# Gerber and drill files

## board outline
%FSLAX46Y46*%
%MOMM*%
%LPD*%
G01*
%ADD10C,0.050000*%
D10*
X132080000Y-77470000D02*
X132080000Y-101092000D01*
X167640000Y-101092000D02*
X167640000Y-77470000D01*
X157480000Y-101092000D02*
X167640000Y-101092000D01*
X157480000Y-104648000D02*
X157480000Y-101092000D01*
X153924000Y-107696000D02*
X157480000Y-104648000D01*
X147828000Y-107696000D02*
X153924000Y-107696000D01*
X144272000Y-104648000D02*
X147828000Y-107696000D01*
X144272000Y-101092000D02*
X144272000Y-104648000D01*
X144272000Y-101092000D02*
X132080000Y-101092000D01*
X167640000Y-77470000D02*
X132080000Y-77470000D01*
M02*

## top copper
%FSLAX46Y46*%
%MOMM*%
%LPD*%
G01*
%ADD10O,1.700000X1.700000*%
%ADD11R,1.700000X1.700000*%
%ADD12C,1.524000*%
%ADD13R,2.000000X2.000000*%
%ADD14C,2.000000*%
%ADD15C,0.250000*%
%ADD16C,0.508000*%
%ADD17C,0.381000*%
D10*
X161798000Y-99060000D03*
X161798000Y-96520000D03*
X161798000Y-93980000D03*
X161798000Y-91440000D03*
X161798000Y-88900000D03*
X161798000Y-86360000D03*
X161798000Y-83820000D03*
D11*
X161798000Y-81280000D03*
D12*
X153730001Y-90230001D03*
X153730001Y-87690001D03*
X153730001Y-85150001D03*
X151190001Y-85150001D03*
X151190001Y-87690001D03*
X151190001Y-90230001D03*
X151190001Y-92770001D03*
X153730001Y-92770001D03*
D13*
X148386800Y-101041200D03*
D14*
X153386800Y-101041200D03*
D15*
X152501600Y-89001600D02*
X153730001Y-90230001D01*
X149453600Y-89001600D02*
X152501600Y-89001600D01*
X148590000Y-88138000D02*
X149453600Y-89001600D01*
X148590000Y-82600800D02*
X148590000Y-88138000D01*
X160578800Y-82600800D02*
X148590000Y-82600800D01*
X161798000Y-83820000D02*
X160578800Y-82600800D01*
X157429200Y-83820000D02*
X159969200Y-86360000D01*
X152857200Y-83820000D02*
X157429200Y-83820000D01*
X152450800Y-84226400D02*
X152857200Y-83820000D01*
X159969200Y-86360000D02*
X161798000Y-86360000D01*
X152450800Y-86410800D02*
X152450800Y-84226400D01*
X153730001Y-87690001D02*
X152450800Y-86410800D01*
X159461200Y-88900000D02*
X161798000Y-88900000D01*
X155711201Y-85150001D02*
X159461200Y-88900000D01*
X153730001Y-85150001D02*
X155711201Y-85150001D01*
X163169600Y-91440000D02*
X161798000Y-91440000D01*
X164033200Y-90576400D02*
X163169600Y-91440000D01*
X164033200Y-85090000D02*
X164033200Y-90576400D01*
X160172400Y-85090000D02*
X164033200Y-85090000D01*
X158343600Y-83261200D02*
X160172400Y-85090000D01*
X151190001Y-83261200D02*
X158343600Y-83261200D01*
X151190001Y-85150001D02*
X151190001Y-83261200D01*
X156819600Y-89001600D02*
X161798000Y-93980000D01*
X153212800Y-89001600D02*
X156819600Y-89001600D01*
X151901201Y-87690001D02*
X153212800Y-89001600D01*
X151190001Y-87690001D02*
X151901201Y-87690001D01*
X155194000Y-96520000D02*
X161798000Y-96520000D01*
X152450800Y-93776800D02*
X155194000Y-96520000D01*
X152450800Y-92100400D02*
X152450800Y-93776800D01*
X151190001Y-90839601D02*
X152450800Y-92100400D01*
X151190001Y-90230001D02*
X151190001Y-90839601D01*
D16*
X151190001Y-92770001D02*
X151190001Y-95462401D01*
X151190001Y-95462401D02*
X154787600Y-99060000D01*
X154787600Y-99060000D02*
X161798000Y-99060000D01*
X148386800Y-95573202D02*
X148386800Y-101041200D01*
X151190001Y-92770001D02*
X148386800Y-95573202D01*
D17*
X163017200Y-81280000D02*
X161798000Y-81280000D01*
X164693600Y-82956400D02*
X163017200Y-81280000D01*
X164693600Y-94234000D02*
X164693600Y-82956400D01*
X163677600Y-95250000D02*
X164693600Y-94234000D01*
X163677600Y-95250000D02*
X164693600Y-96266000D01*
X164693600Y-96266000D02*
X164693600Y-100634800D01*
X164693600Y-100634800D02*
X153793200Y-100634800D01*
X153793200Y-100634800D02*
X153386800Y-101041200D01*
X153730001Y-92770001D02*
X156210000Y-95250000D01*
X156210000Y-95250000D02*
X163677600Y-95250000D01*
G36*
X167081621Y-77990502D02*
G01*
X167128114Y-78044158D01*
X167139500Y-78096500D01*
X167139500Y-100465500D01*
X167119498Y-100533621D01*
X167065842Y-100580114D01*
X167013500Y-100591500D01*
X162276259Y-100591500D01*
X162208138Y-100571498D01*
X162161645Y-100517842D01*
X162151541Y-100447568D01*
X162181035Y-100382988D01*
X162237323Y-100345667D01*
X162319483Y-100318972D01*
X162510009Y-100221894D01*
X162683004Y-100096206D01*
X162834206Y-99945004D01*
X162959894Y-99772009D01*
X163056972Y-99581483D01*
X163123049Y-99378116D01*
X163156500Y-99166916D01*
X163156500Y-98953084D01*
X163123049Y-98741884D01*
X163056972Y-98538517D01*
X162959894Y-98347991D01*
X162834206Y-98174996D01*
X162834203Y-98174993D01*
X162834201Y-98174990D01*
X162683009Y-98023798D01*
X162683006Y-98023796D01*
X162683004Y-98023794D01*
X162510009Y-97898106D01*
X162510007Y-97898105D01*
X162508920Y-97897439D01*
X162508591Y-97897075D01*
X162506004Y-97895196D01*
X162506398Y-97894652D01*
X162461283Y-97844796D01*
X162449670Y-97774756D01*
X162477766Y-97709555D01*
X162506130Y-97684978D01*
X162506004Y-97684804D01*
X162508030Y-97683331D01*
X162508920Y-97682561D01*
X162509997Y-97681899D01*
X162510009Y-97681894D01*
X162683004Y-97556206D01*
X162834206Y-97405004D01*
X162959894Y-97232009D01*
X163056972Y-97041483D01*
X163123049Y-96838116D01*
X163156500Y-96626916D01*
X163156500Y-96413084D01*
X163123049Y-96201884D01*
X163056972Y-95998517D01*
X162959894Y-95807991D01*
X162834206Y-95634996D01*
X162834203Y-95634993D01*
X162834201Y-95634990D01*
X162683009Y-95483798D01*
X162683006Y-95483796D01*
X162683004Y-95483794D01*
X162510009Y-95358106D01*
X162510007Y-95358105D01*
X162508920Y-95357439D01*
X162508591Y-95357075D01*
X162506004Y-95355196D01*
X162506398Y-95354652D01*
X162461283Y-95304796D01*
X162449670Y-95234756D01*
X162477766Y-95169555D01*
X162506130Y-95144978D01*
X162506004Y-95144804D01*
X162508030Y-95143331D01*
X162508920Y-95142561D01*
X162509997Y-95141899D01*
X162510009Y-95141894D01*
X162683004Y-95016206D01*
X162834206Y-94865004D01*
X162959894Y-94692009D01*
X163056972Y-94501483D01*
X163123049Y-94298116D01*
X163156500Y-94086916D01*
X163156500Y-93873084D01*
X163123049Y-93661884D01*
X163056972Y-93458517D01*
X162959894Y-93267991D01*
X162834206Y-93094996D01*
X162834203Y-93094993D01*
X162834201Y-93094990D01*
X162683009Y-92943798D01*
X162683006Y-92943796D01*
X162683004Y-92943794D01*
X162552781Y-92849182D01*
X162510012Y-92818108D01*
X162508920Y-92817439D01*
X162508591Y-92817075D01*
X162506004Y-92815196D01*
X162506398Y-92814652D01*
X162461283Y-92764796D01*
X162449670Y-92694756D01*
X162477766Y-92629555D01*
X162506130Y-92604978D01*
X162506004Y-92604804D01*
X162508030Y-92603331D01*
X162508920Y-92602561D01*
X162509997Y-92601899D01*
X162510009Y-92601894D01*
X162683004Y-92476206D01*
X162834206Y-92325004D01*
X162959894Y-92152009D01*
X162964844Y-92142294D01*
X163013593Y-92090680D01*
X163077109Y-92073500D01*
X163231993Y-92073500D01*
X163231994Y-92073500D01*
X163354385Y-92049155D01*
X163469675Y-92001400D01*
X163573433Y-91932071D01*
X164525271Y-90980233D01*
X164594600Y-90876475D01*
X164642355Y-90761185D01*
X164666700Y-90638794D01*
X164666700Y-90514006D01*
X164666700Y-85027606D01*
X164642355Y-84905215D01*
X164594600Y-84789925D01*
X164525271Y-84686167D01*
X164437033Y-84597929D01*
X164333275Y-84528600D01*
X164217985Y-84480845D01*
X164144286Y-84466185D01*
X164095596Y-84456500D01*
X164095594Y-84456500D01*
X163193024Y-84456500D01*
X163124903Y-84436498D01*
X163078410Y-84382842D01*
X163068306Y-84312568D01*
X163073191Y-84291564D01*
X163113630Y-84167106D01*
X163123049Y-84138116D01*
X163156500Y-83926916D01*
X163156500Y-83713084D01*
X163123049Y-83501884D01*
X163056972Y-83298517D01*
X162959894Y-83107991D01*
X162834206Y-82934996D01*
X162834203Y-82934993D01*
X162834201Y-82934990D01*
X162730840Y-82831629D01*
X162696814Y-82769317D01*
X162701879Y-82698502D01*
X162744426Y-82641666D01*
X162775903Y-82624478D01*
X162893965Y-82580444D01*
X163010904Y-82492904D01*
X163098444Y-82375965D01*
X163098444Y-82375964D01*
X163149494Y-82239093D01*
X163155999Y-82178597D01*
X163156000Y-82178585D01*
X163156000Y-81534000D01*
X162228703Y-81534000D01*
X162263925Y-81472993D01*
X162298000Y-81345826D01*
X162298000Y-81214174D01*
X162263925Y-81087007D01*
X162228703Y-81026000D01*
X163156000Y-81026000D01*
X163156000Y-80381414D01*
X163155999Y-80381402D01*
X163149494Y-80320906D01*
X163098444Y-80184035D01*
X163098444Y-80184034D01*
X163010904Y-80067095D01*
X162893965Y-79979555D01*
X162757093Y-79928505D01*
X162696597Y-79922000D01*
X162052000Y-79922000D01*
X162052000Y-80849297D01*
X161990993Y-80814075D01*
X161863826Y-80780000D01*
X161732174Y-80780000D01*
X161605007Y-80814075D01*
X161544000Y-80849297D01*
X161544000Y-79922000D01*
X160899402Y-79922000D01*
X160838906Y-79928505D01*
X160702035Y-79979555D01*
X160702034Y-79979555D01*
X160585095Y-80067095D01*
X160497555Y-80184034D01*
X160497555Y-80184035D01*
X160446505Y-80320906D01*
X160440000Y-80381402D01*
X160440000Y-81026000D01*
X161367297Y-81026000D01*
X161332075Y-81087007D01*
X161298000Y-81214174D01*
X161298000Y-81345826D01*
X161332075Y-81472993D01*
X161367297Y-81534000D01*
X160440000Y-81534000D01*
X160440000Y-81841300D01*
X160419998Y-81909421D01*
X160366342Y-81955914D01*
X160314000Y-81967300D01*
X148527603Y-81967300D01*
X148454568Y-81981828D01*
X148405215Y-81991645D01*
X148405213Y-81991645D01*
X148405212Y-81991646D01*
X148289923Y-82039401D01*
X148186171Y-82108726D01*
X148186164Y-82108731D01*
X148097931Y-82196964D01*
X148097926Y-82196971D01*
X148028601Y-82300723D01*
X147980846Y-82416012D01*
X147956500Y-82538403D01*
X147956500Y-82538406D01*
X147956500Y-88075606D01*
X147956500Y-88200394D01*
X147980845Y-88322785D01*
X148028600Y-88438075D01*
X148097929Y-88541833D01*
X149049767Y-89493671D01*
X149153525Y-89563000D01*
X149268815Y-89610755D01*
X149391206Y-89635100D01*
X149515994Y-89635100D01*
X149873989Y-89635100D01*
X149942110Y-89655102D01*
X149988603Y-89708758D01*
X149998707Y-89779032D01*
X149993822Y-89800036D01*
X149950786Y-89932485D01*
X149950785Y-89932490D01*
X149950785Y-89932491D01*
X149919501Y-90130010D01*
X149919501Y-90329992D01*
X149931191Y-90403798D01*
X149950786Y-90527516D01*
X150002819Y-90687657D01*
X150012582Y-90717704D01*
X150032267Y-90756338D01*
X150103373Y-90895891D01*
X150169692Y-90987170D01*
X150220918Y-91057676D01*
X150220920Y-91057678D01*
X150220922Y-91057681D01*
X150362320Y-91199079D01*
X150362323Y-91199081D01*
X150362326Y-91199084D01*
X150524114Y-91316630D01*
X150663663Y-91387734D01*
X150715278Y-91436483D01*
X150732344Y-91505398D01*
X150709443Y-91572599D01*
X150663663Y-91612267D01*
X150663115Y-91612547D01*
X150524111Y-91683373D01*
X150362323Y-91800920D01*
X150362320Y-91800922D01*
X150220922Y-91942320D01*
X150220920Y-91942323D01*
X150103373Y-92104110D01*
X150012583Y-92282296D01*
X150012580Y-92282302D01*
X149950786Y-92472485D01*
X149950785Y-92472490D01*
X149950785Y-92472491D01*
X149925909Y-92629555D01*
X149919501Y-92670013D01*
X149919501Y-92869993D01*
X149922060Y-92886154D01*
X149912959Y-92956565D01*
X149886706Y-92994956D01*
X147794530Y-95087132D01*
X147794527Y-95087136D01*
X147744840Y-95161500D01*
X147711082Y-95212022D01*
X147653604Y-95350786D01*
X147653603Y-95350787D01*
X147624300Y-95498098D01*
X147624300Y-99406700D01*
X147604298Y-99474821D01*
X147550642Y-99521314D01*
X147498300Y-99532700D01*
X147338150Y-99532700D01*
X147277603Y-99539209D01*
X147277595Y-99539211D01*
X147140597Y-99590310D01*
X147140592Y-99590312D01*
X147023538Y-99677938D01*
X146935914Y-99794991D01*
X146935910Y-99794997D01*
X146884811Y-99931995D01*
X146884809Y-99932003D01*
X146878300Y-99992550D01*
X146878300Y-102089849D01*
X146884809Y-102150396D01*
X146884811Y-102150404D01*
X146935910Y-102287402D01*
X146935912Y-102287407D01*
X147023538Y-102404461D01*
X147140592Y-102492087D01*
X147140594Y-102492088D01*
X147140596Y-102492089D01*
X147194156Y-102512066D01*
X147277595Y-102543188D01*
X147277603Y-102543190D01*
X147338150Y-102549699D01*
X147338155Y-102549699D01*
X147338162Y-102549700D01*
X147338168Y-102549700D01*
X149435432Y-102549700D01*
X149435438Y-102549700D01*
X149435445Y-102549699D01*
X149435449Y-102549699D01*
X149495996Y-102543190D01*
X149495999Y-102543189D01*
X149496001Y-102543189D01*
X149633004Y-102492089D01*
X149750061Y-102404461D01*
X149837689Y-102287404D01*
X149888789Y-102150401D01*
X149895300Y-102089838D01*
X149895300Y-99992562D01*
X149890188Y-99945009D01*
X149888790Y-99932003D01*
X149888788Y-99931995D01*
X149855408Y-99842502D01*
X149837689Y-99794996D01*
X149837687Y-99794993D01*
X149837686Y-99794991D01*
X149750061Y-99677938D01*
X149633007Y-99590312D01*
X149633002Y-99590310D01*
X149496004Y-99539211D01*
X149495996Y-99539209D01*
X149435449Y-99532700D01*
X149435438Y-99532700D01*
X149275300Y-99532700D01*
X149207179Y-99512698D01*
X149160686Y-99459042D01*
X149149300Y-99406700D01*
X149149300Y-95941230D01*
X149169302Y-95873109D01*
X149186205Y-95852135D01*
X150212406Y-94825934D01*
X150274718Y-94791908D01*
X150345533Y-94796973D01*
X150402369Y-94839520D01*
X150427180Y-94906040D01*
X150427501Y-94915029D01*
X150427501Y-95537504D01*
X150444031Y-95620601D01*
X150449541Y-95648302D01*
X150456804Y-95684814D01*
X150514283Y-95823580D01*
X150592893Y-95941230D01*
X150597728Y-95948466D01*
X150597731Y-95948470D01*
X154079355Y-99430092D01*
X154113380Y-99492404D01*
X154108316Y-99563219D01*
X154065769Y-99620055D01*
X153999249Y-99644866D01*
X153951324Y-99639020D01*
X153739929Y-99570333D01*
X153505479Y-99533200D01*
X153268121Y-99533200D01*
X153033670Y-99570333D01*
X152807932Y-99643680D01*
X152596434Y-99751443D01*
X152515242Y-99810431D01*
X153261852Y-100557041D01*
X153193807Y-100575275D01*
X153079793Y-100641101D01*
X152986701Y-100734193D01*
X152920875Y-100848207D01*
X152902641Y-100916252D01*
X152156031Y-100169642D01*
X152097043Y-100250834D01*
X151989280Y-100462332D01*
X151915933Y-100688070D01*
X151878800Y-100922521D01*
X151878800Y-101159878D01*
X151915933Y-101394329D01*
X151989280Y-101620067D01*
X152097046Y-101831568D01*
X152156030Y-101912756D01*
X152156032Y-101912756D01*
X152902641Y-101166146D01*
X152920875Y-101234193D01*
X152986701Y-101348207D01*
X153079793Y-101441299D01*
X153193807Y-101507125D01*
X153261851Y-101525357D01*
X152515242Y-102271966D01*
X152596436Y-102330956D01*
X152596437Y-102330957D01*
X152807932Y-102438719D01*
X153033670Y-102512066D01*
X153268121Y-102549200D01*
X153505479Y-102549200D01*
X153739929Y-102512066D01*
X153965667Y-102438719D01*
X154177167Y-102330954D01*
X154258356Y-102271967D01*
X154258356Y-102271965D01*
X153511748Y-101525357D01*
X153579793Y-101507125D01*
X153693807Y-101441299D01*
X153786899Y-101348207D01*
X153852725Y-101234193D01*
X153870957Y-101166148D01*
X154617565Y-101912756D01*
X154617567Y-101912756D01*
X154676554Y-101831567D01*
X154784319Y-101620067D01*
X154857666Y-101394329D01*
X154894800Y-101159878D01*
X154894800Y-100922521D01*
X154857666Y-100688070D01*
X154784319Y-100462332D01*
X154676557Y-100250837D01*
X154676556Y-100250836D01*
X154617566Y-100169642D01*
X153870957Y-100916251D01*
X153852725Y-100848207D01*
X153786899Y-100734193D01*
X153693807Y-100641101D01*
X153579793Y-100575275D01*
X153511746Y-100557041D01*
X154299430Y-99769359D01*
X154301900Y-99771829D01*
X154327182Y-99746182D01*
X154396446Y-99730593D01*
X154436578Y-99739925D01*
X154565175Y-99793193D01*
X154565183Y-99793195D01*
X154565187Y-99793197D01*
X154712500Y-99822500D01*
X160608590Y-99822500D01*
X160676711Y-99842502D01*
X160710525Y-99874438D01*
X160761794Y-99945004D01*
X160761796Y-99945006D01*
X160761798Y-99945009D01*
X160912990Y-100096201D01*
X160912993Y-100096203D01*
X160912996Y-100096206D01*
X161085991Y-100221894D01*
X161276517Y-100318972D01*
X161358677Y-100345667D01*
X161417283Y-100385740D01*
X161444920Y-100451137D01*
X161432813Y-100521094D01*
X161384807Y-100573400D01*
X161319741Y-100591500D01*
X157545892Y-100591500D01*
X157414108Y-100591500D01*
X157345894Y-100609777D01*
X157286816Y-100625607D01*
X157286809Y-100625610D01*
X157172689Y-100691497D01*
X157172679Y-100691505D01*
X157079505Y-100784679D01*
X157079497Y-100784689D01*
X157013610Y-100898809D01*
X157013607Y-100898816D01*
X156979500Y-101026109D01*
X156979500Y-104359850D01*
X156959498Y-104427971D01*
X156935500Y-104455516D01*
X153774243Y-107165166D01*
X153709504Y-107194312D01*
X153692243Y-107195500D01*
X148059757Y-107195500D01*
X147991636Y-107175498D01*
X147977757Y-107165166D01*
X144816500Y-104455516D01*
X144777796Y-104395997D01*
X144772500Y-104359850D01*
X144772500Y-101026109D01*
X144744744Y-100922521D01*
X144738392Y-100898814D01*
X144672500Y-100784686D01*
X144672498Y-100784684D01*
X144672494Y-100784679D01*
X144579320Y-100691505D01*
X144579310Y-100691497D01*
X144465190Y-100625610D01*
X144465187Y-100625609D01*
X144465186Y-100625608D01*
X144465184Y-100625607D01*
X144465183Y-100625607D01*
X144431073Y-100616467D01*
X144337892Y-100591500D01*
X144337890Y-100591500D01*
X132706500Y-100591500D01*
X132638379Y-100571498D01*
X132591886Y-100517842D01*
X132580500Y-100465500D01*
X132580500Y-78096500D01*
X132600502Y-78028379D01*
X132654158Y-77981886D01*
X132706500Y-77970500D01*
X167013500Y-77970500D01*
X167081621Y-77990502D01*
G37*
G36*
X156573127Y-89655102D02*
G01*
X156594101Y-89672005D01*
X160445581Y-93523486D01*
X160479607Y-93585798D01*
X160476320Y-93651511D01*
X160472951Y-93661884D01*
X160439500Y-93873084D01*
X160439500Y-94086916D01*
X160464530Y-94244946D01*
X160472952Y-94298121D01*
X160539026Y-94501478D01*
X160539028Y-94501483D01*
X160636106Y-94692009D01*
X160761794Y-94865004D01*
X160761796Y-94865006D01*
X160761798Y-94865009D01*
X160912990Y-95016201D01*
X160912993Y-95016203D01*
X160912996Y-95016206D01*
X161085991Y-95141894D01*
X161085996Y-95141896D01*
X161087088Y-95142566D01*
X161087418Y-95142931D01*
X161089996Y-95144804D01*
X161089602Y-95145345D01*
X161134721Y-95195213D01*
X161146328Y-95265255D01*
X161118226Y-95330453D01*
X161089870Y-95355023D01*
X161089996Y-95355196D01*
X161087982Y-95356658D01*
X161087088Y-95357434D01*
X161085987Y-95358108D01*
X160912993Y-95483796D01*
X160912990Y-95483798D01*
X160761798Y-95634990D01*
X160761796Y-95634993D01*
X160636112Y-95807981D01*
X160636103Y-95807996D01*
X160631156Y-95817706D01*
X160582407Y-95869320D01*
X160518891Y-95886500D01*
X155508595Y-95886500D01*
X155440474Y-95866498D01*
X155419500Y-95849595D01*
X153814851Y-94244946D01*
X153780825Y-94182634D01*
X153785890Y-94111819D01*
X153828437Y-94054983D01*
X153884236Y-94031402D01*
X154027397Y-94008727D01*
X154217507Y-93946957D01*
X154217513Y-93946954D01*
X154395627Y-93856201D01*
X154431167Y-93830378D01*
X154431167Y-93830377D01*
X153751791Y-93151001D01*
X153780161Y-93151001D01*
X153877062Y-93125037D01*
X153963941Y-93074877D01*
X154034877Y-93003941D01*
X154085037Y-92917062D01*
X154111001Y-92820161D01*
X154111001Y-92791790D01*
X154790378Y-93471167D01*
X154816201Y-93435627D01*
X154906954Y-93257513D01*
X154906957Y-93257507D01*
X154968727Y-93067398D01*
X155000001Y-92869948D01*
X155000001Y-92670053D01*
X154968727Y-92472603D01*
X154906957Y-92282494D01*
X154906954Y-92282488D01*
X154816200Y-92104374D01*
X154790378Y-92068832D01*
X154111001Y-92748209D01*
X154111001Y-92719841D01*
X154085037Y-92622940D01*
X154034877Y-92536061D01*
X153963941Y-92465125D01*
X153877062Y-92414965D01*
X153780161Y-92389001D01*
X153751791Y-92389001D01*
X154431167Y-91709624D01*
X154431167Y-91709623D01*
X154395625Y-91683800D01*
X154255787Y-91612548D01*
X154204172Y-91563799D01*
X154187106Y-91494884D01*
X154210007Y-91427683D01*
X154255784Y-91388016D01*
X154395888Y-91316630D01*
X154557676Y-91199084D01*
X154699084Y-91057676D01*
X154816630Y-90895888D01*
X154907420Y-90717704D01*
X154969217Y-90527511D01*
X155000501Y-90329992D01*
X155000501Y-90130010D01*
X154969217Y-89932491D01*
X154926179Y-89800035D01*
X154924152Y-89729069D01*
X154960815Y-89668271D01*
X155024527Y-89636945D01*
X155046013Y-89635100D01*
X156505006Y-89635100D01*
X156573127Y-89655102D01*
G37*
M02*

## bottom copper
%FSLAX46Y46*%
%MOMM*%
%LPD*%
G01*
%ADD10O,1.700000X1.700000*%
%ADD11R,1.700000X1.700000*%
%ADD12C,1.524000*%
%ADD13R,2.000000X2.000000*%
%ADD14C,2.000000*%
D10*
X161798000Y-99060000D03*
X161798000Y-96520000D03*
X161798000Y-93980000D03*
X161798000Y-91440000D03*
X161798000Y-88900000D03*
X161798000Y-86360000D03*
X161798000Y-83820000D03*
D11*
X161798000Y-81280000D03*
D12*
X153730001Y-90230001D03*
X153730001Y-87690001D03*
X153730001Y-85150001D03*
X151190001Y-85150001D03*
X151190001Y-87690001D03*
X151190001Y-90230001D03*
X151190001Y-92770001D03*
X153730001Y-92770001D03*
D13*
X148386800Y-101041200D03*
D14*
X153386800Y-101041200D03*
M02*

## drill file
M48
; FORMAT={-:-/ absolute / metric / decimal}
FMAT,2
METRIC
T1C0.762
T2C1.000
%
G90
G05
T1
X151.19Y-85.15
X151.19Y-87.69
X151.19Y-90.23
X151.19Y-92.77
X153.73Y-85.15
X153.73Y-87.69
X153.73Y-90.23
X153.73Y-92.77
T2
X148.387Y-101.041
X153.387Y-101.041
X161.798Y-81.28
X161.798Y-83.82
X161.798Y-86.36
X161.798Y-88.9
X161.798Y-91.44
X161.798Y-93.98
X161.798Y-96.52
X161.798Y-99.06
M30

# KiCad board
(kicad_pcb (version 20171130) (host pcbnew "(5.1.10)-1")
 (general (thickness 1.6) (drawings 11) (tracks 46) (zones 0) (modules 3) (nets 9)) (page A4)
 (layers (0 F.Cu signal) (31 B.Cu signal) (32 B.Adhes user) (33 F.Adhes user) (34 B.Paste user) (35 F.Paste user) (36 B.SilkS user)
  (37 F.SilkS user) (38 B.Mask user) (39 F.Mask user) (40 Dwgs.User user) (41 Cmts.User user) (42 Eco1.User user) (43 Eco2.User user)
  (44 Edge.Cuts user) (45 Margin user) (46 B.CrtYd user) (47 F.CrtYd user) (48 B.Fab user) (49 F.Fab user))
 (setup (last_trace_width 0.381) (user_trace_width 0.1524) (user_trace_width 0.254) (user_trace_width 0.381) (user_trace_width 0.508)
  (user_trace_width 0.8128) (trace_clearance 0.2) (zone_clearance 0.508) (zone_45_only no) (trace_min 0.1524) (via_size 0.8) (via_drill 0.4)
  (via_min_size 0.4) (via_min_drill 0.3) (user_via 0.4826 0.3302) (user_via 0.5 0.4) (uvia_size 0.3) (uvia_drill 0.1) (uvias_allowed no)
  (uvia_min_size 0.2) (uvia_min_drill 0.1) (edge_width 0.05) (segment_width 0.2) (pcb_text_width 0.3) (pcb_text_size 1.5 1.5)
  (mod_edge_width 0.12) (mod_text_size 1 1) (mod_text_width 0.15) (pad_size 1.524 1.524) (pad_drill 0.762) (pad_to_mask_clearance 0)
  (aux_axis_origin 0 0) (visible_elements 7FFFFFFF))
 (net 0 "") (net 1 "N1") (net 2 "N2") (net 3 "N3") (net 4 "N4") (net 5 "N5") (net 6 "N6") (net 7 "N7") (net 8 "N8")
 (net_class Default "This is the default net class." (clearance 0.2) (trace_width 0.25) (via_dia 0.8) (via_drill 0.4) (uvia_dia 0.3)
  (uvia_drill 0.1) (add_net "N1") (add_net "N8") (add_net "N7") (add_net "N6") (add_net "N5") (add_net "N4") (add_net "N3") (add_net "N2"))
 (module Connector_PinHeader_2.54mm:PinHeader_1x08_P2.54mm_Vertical (layer F.Cu) (at 161.798 81.28)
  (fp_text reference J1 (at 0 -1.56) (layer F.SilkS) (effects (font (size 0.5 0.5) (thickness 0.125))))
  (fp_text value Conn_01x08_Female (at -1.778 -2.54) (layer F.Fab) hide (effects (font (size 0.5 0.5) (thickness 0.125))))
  (pad 8 thru_hole oval (at 0 17.78) (size 1.7 1.7) (drill 1) (layers *.Cu *.Mask) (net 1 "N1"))
  (pad 7 thru_hole oval (at 0 15.24) (size 1.7 1.7) (drill 1) (layers *.Cu *.Mask) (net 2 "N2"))
  (pad 6 thru_hole oval (at 0 12.7) (size 1.7 1.7) (drill 1) (layers *.Cu *.Mask) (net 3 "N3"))
  (pad 5 thru_hole oval (at 0 10.16) (size 1.7 1.7) (drill 1) (layers *.Cu *.Mask) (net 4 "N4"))
  (pad 4 thru_hole oval (at 0 7.62) (size 1.7 1.7) (drill 1) (layers *.Cu *.Mask) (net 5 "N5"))
  (pad 3 thru_hole oval (at 0 5.08) (size 1.7 1.7) (drill 1) (layers *.Cu *.Mask) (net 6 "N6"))
  (pad 2 thru_hole oval (at 0 2.54) (size 1.7 1.7) (drill 1) (layers *.Cu *.Mask) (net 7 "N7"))
  (pad 1 thru_hole rect (at 0 0) (size 1.7 1.7) (drill 1) (layers *.Cu *.Mask) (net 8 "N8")))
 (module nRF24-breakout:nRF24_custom (layer F.Cu) (at 144.840001 88.960001)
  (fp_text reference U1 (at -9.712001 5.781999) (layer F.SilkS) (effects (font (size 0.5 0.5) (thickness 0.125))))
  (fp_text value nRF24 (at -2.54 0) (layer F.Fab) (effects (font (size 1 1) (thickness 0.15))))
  (pad 1 thru_hole circle (at 8.89 1.27) (size 1.524 1.524) (drill 0.762) (layers *.Cu *.Mask) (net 7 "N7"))
  (pad 2 thru_hole circle (at 8.89 -1.27) (size 1.524 1.524) (drill 0.762) (layers *.Cu *.Mask) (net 6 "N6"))
  (pad 3 thru_hole circle (at 8.89 -3.81) (size 1.524 1.524) (drill 0.762) (layers *.Cu *.Mask) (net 5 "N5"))
  (pad 4 thru_hole circle (at 6.35 -3.81) (size 1.524 1.524) (drill 0.762) (layers *.Cu *.Mask) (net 4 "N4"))
  (pad 5 thru_hole circle (at 6.35 -1.27) (size 1.524 1.524) (drill 0.762) (layers *.Cu *.Mask) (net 3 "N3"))
  (pad 6 thru_hole circle (at 6.35 1.27) (size 1.524 1.524) (drill 0.762) (layers *.Cu *.Mask) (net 2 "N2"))
  (pad 7 thru_hole circle (at 6.35 3.81) (size 1.524 1.524) (drill 0.762) (layers *.Cu *.Mask) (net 1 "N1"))
  (pad 0 thru_hole circle (at 8.89 3.81) (size 1.524 1.524) (drill 0.762) (layers *.Cu *.Mask) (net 8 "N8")))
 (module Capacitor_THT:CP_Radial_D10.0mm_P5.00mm (layer F.Cu) (at 148.3868 101.0412)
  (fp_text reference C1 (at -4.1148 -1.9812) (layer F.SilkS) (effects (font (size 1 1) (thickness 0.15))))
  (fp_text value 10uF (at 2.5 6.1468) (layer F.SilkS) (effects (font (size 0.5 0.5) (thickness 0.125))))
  (pad 1 thru_hole rect (at 0 0) (size 2 2) (drill 1) (layers *.Cu *.Mask) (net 1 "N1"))
  (pad 2 thru_hole circle (at 5 0) (size 2 2) (drill 1) (layers *.Cu *.Mask) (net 8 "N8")))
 (gr_line (start 132.08 77.47) (end 132.08 101.092) (layer Edge.Cuts) (width 0.05))
 (gr_line (start 167.64 101.092) (end 167.64 77.47) (layer Edge.Cuts) (width 0.05))
 (gr_line (start 157.48 101.092) (end 167.64 101.092) (layer Edge.Cuts) (width 0.05))
 (gr_line (start 157.48 104.648) (end 157.48 101.092) (layer Edge.Cuts) (width 0.05))
 (gr_line (start 153.924 107.696) (end 157.48 104.648) (layer Edge.Cuts) (width 0.05))
 (gr_line (start 147.828 107.696) (end 153.924 107.696) (layer Edge.Cuts) (width 0.05))
 (gr_line (start 144.272 104.648) (end 147.828 107.696) (layer Edge.Cuts) (width 0.05))
 (gr_line (start 144.272 101.092) (end 144.272 104.648) (layer Edge.Cuts) (width 0.05))
 (gr_line (start 144.272 101.092) (end 132.08 101.092) (layer Edge.Cuts) (width 0.05))
 (gr_line (start 167.64 77.47) (end 132.08 77.47) (layer Edge.Cuts) (width 0.05))
 (segment (start 152.5016 89.0016) (end 153.730001 90.230001) (width 0.25) (layer F.Cu) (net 7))
 (segment (start 149.4536 89.0016) (end 152.5016 89.0016) (width 0.25) (layer F.Cu) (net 7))
 (segment (start 148.59 88.138) (end 149.4536 89.0016) (width 0.25) (layer F.Cu) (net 7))
 (segment (start 148.59 82.6008) (end 148.59 88.138) (width 0.25) (layer F.Cu) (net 7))
 (segment (start 160.5788 82.6008) (end 148.59 82.6008) (width 0.25) (layer F.Cu) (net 7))
 (segment (start 161.798 83.82) (end 160.5788 82.6008) (width 0.25) (layer F.Cu) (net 7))
 (segment (start 157.4292 83.82) (end 159.9692 86.36) (width 0.25) (layer F.Cu) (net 6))
 (segment (start 152.8572 83.82) (end 157.4292 83.82) (width 0.25) (layer F.Cu) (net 6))
 (segment (start 152.4508 84.2264) (end 152.8572 83.82) (width 0.25) (layer F.Cu) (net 6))
 (segment (start 159.9692 86.36) (end 161.798 86.36) (width 0.25) (layer F.Cu) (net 6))
 (segment (start 152.4508 86.4108) (end 152.4508 84.2264) (width 0.25) (layer F.Cu) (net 6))
 (segment (start 153.730001 87.690001) (end 152.4508 86.4108) (width 0.25) (layer F.Cu) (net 6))
 (segment (start 159.4612 88.9) (end 161.798 88.9) (width 0.25) (layer F.Cu) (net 5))
 (segment (start 155.711201 85.150001) (end 159.4612 88.9) (width 0.25) (layer F.Cu) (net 5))
 (segment (start 153.730001 85.150001) (end 155.711201 85.150001) (width 0.25) (layer F.Cu) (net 5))
 (segment (start 163.1696 91.44) (end 161.798 91.44) (width 0.25) (layer F.Cu) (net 4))
 (segment (start 164.0332 90.5764) (end 163.1696 91.44) (width 0.25) (layer F.Cu) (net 4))
 (segment (start 164.0332 85.09) (end 164.0332 90.5764) (width 0.25) (layer F.Cu) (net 4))
 (segment (start 160.1724 85.09) (end 164.0332 85.09) (width 0.25) (layer F.Cu) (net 4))
 (segment (start 158.3436 83.2612) (end 160.1724 85.09) (width 0.25) (layer F.Cu) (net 4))
 (segment (start 151.190001 83.2612) (end 158.3436 83.2612) (width 0.25) (layer F.Cu) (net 4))
 (segment (start 151.190001 85.150001) (end 151.190001 83.2612) (width 0.25) (layer F.Cu) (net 4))
 (segment (start 156.8196 89.0016) (end 161.798 93.98) (width 0.25) (layer F.Cu) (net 3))
 (segment (start 153.2128 89.0016) (end 156.8196 89.0016) (width 0.25) (layer F.Cu) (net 3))
 (segment (start 151.901201 87.690001) (end 153.2128 89.0016) (width 0.25) (layer F.Cu) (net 3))
 (segment (start 151.190001 87.690001) (end 151.901201 87.690001) (width 0.25) (layer F.Cu) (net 3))
 (segment (start 155.194 96.52) (end 161.798 96.52) (width 0.25) (layer F.Cu) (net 2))
 (segment (start 152.4508 93.7768) (end 155.194 96.52) (width 0.25) (layer F.Cu) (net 2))
 (segment (start 152.4508 92.1004) (end 152.4508 93.7768) (width 0.25) (layer F.Cu) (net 2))
 (segment (start 151.190001 90.839601) (end 152.4508 92.1004) (width 0.25) (layer F.Cu) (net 2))
 (segment (start 151.190001 90.230001) (end 151.190001 90.839601) (width 0.25) (layer F.Cu) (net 2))
 (segment (start 151.190001 92.770001) (end 151.190001 95.462401) (width 0.508) (layer F.Cu) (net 1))
 (segment (start 151.190001 95.462401) (end 154.7876 99.06) (width 0.508) (layer F.Cu) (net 1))
 (segment (start 154.7876 99.06) (end 161.798 99.06) (width 0.508) (layer F.Cu) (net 1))
 (segment (start 148.3868 95.573202) (end 148.3868 101.0412) (width 0.508) (layer F.Cu) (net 1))
 (segment (start 151.190001 92.770001) (end 148.3868 95.573202) (width 0.508) (layer F.Cu) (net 1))
 (segment (start 163.0172 81.28) (end 161.798 81.28) (width 0.381) (layer F.Cu) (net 8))
 (segment (start 164.6936 82.9564) (end 163.0172 81.28) (width 0.381) (layer F.Cu) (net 8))
 (segment (start 164.6936 94.234) (end 164.6936 82.9564) (width 0.381) (layer F.Cu) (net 8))
 (segment (start 163.6776 95.25) (end 164.6936 94.234) (width 0.381) (layer F.Cu) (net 8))
 (segment (start 163.6776 95.25) (end 164.6936 96.266) (width 0.381) (layer F.Cu) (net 8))
 (segment (start 164.6936 96.266) (end 164.6936 100.6348) (width 0.381) (layer F.Cu) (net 8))
 (segment (start 164.6936 100.6348) (end 153.7932 100.6348) (width 0.381) (layer F.Cu) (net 8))
 (segment (start 153.7932 100.6348) (end 153.3868 101.0412) (width 0.381) (layer F.Cu) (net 8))
 (segment (start 153.730001 92.770001) (end 156.21 95.25) (width 0.381) (layer F.Cu) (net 8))
 (segment (start 156.21 95.25) (end 163.6776 95.25) (width 0.381) (layer F.Cu) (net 8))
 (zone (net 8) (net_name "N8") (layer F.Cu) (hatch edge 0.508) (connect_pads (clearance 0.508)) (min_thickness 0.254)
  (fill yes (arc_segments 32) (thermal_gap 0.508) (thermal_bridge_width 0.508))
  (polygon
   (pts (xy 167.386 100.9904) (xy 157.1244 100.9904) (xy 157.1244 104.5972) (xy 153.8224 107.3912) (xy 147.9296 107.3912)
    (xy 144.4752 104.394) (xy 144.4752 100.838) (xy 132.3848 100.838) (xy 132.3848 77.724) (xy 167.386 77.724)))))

